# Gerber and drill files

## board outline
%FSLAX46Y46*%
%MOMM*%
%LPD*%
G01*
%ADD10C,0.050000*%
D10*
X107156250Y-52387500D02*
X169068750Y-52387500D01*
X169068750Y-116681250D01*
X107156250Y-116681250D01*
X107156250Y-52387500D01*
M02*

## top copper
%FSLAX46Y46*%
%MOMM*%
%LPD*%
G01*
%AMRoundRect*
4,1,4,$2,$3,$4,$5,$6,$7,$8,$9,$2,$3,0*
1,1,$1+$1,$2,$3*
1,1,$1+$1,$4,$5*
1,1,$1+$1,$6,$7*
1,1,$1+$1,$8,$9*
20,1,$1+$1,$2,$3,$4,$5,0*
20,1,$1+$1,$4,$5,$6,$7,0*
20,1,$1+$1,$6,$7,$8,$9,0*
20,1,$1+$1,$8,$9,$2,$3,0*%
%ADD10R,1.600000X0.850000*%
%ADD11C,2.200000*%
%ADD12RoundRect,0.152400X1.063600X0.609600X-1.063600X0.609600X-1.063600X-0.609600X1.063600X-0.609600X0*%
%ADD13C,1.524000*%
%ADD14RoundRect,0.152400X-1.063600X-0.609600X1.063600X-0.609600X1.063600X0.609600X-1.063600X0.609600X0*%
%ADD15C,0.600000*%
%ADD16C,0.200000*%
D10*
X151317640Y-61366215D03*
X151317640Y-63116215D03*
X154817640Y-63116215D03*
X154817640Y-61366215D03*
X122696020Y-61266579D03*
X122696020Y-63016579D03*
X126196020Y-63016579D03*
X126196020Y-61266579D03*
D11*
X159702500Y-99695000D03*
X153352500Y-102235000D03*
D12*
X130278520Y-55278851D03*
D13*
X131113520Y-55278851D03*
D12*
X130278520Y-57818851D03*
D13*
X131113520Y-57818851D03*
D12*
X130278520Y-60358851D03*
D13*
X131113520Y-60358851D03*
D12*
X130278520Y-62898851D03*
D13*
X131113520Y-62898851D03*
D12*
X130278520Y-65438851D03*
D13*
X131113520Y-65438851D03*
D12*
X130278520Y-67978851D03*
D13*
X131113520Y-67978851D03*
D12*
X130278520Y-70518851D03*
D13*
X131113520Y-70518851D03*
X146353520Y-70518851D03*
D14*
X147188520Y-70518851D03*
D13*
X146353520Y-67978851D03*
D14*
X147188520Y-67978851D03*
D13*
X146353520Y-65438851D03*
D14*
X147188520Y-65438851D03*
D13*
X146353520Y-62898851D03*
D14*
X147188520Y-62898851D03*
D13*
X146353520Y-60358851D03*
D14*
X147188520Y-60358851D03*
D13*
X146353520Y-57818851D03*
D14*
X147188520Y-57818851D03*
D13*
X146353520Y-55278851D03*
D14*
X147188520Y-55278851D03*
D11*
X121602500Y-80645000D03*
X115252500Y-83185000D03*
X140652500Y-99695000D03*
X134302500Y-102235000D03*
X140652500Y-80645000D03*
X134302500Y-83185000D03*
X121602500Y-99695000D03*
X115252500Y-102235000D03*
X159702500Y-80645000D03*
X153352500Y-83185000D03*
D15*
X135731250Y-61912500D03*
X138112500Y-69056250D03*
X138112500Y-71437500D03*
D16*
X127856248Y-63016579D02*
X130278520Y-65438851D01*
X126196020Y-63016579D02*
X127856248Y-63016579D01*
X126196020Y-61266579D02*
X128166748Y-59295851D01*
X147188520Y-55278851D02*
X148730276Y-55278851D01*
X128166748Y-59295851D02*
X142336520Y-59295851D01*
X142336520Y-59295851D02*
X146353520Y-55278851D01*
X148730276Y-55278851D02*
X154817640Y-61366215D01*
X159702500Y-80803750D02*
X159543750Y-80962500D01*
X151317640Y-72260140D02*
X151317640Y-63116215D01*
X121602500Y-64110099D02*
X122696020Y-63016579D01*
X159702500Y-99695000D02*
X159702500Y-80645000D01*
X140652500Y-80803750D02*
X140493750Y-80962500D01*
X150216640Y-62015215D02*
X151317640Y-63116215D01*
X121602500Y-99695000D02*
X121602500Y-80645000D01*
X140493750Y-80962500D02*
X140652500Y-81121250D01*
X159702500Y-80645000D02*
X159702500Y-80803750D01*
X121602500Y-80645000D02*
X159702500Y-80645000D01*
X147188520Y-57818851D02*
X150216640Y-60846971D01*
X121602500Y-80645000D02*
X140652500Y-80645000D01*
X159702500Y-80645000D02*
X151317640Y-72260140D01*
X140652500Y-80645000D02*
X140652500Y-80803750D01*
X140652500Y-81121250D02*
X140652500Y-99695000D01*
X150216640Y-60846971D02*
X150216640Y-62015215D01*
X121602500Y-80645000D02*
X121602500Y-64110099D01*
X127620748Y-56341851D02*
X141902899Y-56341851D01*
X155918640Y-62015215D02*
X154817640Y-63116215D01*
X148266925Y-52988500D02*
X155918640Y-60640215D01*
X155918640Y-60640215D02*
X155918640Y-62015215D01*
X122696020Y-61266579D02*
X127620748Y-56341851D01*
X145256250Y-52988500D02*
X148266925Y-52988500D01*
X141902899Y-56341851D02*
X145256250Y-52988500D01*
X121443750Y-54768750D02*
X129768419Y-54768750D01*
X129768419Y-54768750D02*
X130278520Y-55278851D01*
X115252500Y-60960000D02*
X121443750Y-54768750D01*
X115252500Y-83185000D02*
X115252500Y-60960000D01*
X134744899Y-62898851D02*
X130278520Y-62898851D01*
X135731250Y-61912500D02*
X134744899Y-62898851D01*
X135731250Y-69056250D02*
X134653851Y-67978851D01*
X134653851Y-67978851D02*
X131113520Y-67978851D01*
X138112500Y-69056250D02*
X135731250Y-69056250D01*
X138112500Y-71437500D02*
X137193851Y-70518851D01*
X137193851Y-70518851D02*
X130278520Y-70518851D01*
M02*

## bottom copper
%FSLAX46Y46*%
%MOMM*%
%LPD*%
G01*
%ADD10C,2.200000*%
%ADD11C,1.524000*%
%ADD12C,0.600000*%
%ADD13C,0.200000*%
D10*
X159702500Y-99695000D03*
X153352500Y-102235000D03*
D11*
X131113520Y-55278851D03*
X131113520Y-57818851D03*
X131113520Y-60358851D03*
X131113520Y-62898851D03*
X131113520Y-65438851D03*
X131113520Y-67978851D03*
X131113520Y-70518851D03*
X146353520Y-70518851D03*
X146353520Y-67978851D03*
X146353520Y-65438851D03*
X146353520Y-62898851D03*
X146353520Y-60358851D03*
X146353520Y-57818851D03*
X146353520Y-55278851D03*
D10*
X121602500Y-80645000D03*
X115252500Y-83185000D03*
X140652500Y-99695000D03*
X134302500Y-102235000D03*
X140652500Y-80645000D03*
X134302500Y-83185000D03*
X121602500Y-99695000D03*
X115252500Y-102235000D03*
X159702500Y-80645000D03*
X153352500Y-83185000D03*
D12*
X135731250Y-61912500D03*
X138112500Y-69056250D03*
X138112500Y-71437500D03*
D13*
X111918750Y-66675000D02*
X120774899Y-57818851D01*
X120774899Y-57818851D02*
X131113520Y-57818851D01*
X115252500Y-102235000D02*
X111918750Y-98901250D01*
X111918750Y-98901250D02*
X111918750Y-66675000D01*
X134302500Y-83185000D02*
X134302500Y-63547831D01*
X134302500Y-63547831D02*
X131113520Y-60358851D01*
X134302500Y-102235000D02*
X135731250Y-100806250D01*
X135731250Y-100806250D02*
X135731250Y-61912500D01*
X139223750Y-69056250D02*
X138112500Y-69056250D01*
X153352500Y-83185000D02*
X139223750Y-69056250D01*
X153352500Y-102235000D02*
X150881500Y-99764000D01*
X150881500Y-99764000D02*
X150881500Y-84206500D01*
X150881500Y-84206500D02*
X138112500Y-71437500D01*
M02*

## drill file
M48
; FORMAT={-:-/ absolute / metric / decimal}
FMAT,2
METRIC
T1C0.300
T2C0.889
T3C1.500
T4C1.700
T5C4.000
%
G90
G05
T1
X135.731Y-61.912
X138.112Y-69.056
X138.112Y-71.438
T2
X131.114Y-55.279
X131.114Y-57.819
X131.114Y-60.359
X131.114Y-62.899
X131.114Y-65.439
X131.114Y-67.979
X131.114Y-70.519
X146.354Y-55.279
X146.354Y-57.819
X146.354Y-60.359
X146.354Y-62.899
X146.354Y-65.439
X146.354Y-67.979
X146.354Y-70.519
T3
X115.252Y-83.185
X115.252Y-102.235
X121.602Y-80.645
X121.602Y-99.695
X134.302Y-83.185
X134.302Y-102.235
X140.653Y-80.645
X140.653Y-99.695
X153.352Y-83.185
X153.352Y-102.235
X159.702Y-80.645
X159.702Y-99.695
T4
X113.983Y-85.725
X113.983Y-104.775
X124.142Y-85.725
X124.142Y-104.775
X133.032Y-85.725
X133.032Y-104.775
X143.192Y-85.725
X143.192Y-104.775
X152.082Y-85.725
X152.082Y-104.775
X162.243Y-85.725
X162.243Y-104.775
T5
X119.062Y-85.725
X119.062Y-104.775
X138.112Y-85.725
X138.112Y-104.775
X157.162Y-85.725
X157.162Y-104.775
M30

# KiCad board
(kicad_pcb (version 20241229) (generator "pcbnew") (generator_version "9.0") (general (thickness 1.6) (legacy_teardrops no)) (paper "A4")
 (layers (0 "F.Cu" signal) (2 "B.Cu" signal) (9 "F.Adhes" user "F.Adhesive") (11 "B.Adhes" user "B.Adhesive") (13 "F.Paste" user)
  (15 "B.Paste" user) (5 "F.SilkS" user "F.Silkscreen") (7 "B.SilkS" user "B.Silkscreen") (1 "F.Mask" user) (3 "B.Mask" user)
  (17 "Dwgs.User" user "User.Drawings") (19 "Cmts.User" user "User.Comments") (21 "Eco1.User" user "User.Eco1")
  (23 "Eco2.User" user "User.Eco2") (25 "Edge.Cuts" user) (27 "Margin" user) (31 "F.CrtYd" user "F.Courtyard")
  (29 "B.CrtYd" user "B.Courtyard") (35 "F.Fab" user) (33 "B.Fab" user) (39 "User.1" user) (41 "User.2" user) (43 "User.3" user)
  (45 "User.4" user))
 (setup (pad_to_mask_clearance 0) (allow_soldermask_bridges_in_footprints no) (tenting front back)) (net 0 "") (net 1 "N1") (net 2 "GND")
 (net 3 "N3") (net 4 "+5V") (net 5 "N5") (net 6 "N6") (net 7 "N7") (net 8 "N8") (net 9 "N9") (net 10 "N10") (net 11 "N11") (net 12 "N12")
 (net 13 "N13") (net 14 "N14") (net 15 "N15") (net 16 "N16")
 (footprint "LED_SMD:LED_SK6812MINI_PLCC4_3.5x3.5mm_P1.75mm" (layer "F.Cu") (at 153.06764 62.241215)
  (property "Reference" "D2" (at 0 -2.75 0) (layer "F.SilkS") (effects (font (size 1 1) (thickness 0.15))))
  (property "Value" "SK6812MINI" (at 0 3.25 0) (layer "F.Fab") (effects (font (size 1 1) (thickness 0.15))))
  (pad "1" smd rect (at -1.75 -0.875) (size 1.6 0.85) (layers "F.Cu" "F.Mask" "F.Paste") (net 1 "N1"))
  (pad "2" smd rect (at -1.75 0.875) (size 1.6 0.85) (layers "F.Cu" "F.Mask" "F.Paste") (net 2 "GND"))
  (pad "3" smd rect (at 1.75 0.875) (size 1.6 0.85) (layers "F.Cu" "F.Mask" "F.Paste") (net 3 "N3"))
  (pad "4" smd rect (at 1.75 -0.875) (size 1.6 0.85) (layers "F.Cu" "F.Mask" "F.Paste") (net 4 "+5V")))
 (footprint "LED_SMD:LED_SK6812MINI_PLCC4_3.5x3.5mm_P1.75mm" (layer "F.Cu") (at 124.44602 62.141579)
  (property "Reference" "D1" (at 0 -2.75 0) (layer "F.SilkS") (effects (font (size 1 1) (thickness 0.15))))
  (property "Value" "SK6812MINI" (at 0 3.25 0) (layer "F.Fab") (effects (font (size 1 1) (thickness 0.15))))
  (pad "1" smd rect (at -1.75 -0.875) (size 1.6 0.85) (layers "F.Cu" "F.Mask" "F.Paste") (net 3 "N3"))
  (pad "2" smd rect (at -1.75 0.875) (size 1.6 0.85) (layers "F.Cu" "F.Mask" "F.Paste") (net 2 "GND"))
  (pad "3" smd rect (at 1.75 0.875) (size 1.6 0.85) (layers "F.Cu" "F.Mask" "F.Paste") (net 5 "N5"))
  (pad "4" smd rect (at 1.75 -0.875) (size 1.6 0.85) (layers "F.Cu" "F.Mask" "F.Paste") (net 4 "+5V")))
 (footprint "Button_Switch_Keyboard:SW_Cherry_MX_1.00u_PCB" (layer "F.Cu") (at 159.7025 99.695)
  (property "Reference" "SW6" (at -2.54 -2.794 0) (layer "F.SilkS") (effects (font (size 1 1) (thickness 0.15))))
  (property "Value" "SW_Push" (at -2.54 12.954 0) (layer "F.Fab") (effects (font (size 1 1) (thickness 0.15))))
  (pad "" np_thru_hole circle (at -7.62 5.08) (size 1.7 1.7) (drill 1.7) (layers "*.Cu" "*.Mask"))
  (pad "" np_thru_hole circle (at -2.54 5.08) (size 4 4) (drill 4) (layers "*.Cu" "*.Mask"))
  (pad "" np_thru_hole circle (at 2.54 5.08) (size 1.7 1.7) (drill 1.7) (layers "*.Cu" "*.Mask"))
  (pad "1" thru_hole circle (at 0 0) (size 2.2 2.2) (drill 1.5) (layers "*.Cu" "*.Mask") (remove_unused_layers no) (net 2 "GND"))
  (pad "2" thru_hole circle (at -6.35 2.54) (size 2.2 2.2) (drill 1.5) (layers "*.Cu" "*.Mask") (remove_unused_layers no) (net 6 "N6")))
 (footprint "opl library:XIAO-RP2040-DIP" (layer "F.Cu") (at 138.73352 62.898851)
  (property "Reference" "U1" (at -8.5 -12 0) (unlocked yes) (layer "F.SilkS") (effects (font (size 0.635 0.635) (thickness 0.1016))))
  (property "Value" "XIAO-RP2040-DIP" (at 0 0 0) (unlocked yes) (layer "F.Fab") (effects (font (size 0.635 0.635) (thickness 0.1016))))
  (pad "1" smd roundrect (at -8.455 -7.62 180) (size 2.432 1.524) (layers "F.Cu" "F.Mask") (roundrect_rratio 0.1) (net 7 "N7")
   (thermal_bridge_angle 45))
  (pad "1" thru_hole circle (at -7.62 -7.62 180) (size 1.524 1.524) (drill 0.889) (layers "*.Cu" "*.Mask") (remove_unused_layers no)
   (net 7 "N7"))
  (pad "2" smd roundrect (at -8.455 -5.08 180) (size 2.432 1.524) (layers "F.Cu" "F.Mask") (roundrect_rratio 0.1) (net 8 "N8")
   (thermal_bridge_angle 45))
  (pad "2" thru_hole circle (at -7.62 -5.08 180) (size 1.524 1.524) (drill 0.889) (layers "*.Cu" "*.Mask") (remove_unused_layers no)
   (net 8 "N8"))
  (pad "3" smd roundrect (at -8.455 -2.54 180) (size 2.432 1.524) (layers "F.Cu" "F.Mask") (roundrect_rratio 0.1) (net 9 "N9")
   (thermal_bridge_angle 45))
  (pad "3" thru_hole circle (at -7.62 -2.54 180) (size 1.524 1.524) (drill 0.889) (layers "*.Cu" "*.Mask") (remove_unused_layers no)
   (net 9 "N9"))
  (pad "4" smd roundrect (at -8.455 0 180) (size 2.432 1.524) (layers "F.Cu" "F.Mask") (roundrect_rratio 0.1) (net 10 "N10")
   (thermal_bridge_angle 45))
  (pad "4" thru_hole circle (at -7.62 0 180) (size 1.524 1.524) (drill 0.889) (layers "*.Cu" "*.Mask") (remove_unused_layers no)
   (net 10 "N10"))
  (pad "5" smd roundrect (at -8.455 2.54 180) (size 2.432 1.524) (layers "F.Cu" "F.Mask") (roundrect_rratio 0.1) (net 5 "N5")
   (thermal_bridge_angle 45))
  (pad "5" thru_hole circle (at -7.62 2.54 180) (size 1.524 1.524) (drill 0.889) (layers "*.Cu" "*.Mask") (remove_unused_layers no)
   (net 5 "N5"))
  (pad "6" smd roundrect (at -8.455 5.08 180) (size 2.432 1.524) (layers "F.Cu" "F.Mask") (roundrect_rratio 0.1) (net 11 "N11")
   (thermal_bridge_angle 45))
  (pad "6" thru_hole circle (at -7.62 5.08 180) (size 1.524 1.524) (drill 0.889) (layers "*.Cu" "*.Mask") (remove_unused_layers no)
   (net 11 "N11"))
  (pad "7" smd roundrect (at -8.455 7.62 180) (size 2.432 1.524) (layers "F.Cu" "F.Mask") (roundrect_rratio 0.1) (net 6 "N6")
   (thermal_bridge_angle 45))
  (pad "7" thru_hole circle (at -7.62 7.62 180) (size 1.524 1.524) (drill 0.889) (layers "*.Cu" "*.Mask") (remove_unused_layers no)
   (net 6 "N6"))
  (pad "8" thru_hole circle (at 7.62 7.62) (size 1.524 1.524) (drill 0.889) (layers "*.Cu" "*.Mask") (remove_unused_layers no)
   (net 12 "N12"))
  (pad "8" smd roundrect (at 8.455 7.62) (size 2.432 1.524) (layers "F.Cu" "F.Mask") (roundrect_rratio 0.1) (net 12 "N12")
   (thermal_bridge_angle 45))
  (pad "9" thru_hole circle (at 7.62 5.08) (size 1.524 1.524) (drill 0.889) (layers "*.Cu" "*.Mask") (remove_unused_layers no)
   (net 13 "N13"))
  (pad "9" smd roundrect (at 8.455 5.08) (size 2.432 1.524) (layers "F.Cu" "F.Mask") (roundrect_rratio 0.1) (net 13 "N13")
   (thermal_bridge_angle 45))
  (pad "10" thru_hole circle (at 7.62 2.54) (size 1.524 1.524) (drill 0.889) (layers "*.Cu" "*.Mask") (remove_unused_layers no)
   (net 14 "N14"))
  (pad "10" smd roundrect (at 8.455 2.54) (size 2.432 1.524) (layers "F.Cu" "F.Mask") (roundrect_rratio 0.1) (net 14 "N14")
   (thermal_bridge_angle 45))
  (pad "11" thru_hole circle (at 7.62 0) (size 1.524 1.524) (drill 0.889) (layers "*.Cu" "*.Mask") (remove_unused_layers no) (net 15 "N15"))
  (pad "11" smd roundrect (at 8.455 0) (size 2.432 1.524) (layers "F.Cu" "F.Mask") (roundrect_rratio 0.1) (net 15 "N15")
   (thermal_bridge_angle 45))
  (pad "12" thru_hole circle (at 7.62 -2.54) (size 1.524 1.524) (drill 0.889) (layers "*.Cu" "*.Mask") (remove_unused_layers no)
   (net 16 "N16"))
  (pad "12" smd roundrect (at 8.455 -2.54) (size 2.432 1.524) (layers "F.Cu" "F.Mask") (roundrect_rratio 0.1) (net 16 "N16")
   (thermal_bridge_angle 45))
  (pad "13" thru_hole circle (at 7.62 -5.08) (size 1.524 1.524) (drill 0.889) (layers "*.Cu" "*.Mask") (remove_unused_layers no)
   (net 2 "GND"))
  (pad "13" smd roundrect (at 8.455 -5.08) (size 2.432 1.524) (layers "F.Cu" "F.Mask") (roundrect_rratio 0.1) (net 2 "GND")
   (thermal_bridge_angle 45))
  (pad "14" thru_hole circle (at 7.62 -7.62) (size 1.524 1.524) (drill 0.889) (layers "*.Cu" "*.Mask") (remove_unused_layers no)
   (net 4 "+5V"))
  (pad "14" smd roundrect (at 8.455 -7.62) (size 2.432 1.524) (layers "F.Cu" "F.Mask") (roundrect_rratio 0.1) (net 4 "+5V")
   (thermal_bridge_angle 45)))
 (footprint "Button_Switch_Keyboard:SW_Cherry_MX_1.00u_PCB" (layer "F.Cu") (at 121.6025 80.645)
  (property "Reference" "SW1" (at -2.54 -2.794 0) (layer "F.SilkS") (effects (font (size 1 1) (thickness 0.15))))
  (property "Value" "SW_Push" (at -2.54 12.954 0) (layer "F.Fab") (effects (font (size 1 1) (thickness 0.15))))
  (pad "" np_thru_hole circle (at -7.62 5.08) (size 1.7 1.7) (drill 1.7) (layers "*.Cu" "*.Mask"))
  (pad "" np_thru_hole circle (at -2.54 5.08) (size 4 4) (drill 4) (layers "*.Cu" "*.Mask"))
  (pad "" np_thru_hole circle (at 2.54 5.08) (size 1.7 1.7) (drill 1.7) (layers "*.Cu" "*.Mask"))
  (pad "1" thru_hole circle (at 0 0) (size 2.2 2.2) (drill 1.5) (layers "*.Cu" "*.Mask") (remove_unused_layers no) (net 2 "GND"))
  (pad "2" thru_hole circle (at -6.35 2.54) (size 2.2 2.2) (drill 1.5) (layers "*.Cu" "*.Mask") (remove_unused_layers no) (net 7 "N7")))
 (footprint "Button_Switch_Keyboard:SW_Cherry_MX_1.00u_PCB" (layer "F.Cu") (at 140.6525 99.695)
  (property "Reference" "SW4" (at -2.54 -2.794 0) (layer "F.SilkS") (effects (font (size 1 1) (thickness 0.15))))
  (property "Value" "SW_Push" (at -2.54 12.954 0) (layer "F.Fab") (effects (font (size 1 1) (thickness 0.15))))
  (pad "" np_thru_hole circle (at -7.62 5.08) (size 1.7 1.7) (drill 1.7) (layers "*.Cu" "*.Mask"))
  (pad "" np_thru_hole circle (at -2.54 5.08) (size 4 4) (drill 4) (layers "*.Cu" "*.Mask"))
  (pad "" np_thru_hole circle (at 2.54 5.08) (size 1.7 1.7) (drill 1.7) (layers "*.Cu" "*.Mask"))
  (pad "1" thru_hole circle (at 0 0) (size 2.2 2.2) (drill 1.5) (layers "*.Cu" "*.Mask") (remove_unused_layers no) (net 2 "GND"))
  (pad "2" thru_hole circle (at -6.35 2.54) (size 2.2 2.2) (drill 1.5) (layers "*.Cu" "*.Mask") (remove_unused_layers no) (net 10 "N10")))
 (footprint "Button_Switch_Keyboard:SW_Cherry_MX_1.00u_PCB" (layer "F.Cu") (at 140.6525 80.645)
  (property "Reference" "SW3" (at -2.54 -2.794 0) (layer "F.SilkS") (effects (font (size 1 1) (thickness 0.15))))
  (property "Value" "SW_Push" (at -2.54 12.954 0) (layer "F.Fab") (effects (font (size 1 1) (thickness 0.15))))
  (pad "" np_thru_hole circle (at -7.62 5.08) (size 1.7 1.7) (drill 1.7) (layers "*.Cu" "*.Mask"))
  (pad "" np_thru_hole circle (at -2.54 5.08) (size 4 4) (drill 4) (layers "*.Cu" "*.Mask"))
  (pad "" np_thru_hole circle (at 2.54 5.08) (size 1.7 1.7) (drill 1.7) (layers "*.Cu" "*.Mask"))
  (pad "1" thru_hole circle (at 0 0) (size 2.2 2.2) (drill 1.5) (layers "*.Cu" "*.Mask") (remove_unused_layers no) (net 2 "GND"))
  (pad "2" thru_hole circle (at -6.35 2.54) (size 2.2 2.2) (drill 1.5) (layers "*.Cu" "*.Mask") (remove_unused_layers no) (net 9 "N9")))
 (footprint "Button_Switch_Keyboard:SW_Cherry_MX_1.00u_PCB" (layer "F.Cu") (at 121.6025 99.695)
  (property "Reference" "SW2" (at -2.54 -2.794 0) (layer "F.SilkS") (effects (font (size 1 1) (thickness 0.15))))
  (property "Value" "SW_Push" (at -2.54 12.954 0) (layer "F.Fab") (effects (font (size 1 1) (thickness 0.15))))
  (pad "" np_thru_hole circle (at -7.62 5.08) (size 1.7 1.7) (drill 1.7) (layers "*.Cu" "*.Mask"))
  (pad "" np_thru_hole circle (at -2.54 5.08) (size 4 4) (drill 4) (layers "*.Cu" "*.Mask"))
  (pad "" np_thru_hole circle (at 2.54 5.08) (size 1.7 1.7) (drill 1.7) (layers "*.Cu" "*.Mask"))
  (pad "1" thru_hole circle (at 0 0) (size 2.2 2.2) (drill 1.5) (layers "*.Cu" "*.Mask") (remove_unused_layers no) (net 2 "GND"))
  (pad "2" thru_hole circle (at -6.35 2.54) (size 2.2 2.2) (drill 1.5) (layers "*.Cu" "*.Mask") (remove_unused_layers no) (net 8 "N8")))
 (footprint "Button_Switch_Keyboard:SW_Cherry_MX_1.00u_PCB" (layer "F.Cu") (at 159.7025 80.645)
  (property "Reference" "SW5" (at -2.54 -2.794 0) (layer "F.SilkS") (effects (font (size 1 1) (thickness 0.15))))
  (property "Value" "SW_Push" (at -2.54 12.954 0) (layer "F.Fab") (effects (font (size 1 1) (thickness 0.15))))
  (pad "" np_thru_hole circle (at -7.62 5.08) (size 1.7 1.7) (drill 1.7) (layers "*.Cu" "*.Mask"))
  (pad "" np_thru_hole circle (at -2.54 5.08) (size 4 4) (drill 4) (layers "*.Cu" "*.Mask"))
  (pad "" np_thru_hole circle (at 2.54 5.08) (size 1.7 1.7) (drill 1.7) (layers "*.Cu" "*.Mask"))
  (pad "1" thru_hole circle (at 0 0) (size 2.2 2.2) (drill 1.5) (layers "*.Cu" "*.Mask") (remove_unused_layers no) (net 2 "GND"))
  (pad "2" thru_hole circle (at -6.35 2.54) (size 2.2 2.2) (drill 1.5) (layers "*.Cu" "*.Mask") (remove_unused_layers no) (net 11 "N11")))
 (gr_rect (start 107.15625 52.3875) (end 169.06875 116.68125) (stroke (width 0.05) (type default)) (fill no) (layer "Edge.Cuts"))
 (segment (start 127.856248 63.016579) (end 130.27852 65.438851) (width 0.2) (layer "F.Cu") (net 5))
 (segment (start 126.19602 63.016579) (end 127.856248 63.016579) (width 0.2) (layer "F.Cu") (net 5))
 (segment (start 126.19602 61.266579) (end 128.166748 59.295851) (width 0.2) (layer "F.Cu") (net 4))
 (segment (start 147.18852 55.278851) (end 148.730276 55.278851) (width 0.2) (layer "F.Cu") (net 4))
 (segment (start 128.166748 59.295851) (end 142.33652 59.295851) (width 0.2) (layer "F.Cu") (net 4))
 (segment (start 142.33652 59.295851) (end 146.35352 55.278851) (width 0.2) (layer "F.Cu") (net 4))
 (segment (start 148.730276 55.278851) (end 154.81764 61.366215) (width 0.2) (layer "F.Cu") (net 4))
 (segment (start 159.7025 80.80375) (end 159.54375 80.9625) (width 0.2) (layer "F.Cu") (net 2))
 (segment (start 151.31764 72.26014) (end 151.31764 63.116215) (width 0.2) (layer "F.Cu") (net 2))
 (segment (start 121.6025 64.110099) (end 122.69602 63.016579) (width 0.2) (layer "F.Cu") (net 2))
 (segment (start 159.7025 99.695) (end 159.7025 80.645) (width 0.2) (layer "F.Cu") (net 2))
 (segment (start 140.6525 80.80375) (end 140.49375 80.9625) (width 0.2) (layer "F.Cu") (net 2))
 (segment (start 150.21664 62.015215) (end 151.31764 63.116215) (width 0.2) (layer "F.Cu") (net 2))
 (segment (start 121.6025 99.695) (end 121.6025 80.645) (width 0.2) (layer "F.Cu") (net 2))
 (segment (start 140.49375 80.9625) (end 140.6525 81.12125) (width 0.2) (layer "F.Cu") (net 2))
 (segment (start 159.7025 80.645) (end 159.7025 80.80375) (width 0.2) (layer "F.Cu") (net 2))
 (segment (start 121.6025 80.645) (end 159.7025 80.645) (width 0.2) (layer "F.Cu") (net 2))
 (segment (start 147.18852 57.818851) (end 150.21664 60.846971) (width 0.2) (layer "F.Cu") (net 2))
 (segment (start 121.6025 80.645) (end 140.6525 80.645) (width 0.2) (layer "F.Cu") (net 2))
 (segment (start 159.7025 80.645) (end 151.31764 72.26014) (width 0.2) (layer "F.Cu") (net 2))
 (segment (start 140.6525 80.645) (end 140.6525 80.80375) (width 0.2) (layer "F.Cu") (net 2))
 (segment (start 140.6525 81.12125) (end 140.6525 99.695) (width 0.2) (layer "F.Cu") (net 2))
 (segment (start 150.21664 60.846971) (end 150.21664 62.015215) (width 0.2) (layer "F.Cu") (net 2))
 (segment (start 121.6025 80.645) (end 121.6025 64.110099) (width 0.2) (layer "F.Cu") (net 2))
 (segment (start 127.620748 56.341851) (end 141.902899 56.341851) (width 0.2) (layer "F.Cu") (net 3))
 (segment (start 155.91864 62.015215) (end 154.81764 63.116215) (width 0.2) (layer "F.Cu") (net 3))
 (segment (start 148.266925 52.9885) (end 155.91864 60.640215) (width 0.2) (layer "F.Cu") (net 3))
 (segment (start 155.91864 60.640215) (end 155.91864 62.015215) (width 0.2) (layer "F.Cu") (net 3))
 (segment (start 122.69602 61.266579) (end 127.620748 56.341851) (width 0.2) (layer "F.Cu") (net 3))
 (segment (start 145.25625 52.9885) (end 148.266925 52.9885) (width 0.2) (layer "F.Cu") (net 3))
 (segment (start 141.902899 56.341851) (end 145.25625 52.9885) (width 0.2) (layer "F.Cu") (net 3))
 (segment (start 121.44375 54.76875) (end 129.768419 54.76875) (width 0.2) (layer "F.Cu") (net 7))
 (segment (start 129.768419 54.76875) (end 130.27852 55.278851) (width 0.2) (layer "F.Cu") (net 7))
 (segment (start 115.2525 60.96) (end 121.44375 54.76875) (width 0.2) (layer "F.Cu") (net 7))
 (segment (start 115.2525 83.185) (end 115.2525 60.96) (width 0.2) (layer "F.Cu") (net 7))
 (segment (start 111.91875 66.675) (end 120.774899 57.818851) (width 0.2) (layer "B.Cu") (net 8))
 (segment (start 120.774899 57.818851) (end 131.11352 57.818851) (width 0.2) (layer "B.Cu") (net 8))
 (segment (start 115.2525 102.235) (end 111.91875 98.90125) (width 0.2) (layer "B.Cu") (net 8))
 (segment (start 111.91875 98.90125) (end 111.91875 66.675) (width 0.2) (layer "B.Cu") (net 8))
 (segment (start 134.3025 83.185) (end 134.3025 63.547831) (width 0.2) (layer "B.Cu") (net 9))
 (segment (start 134.3025 63.547831) (end 131.11352 60.358851) (width 0.2) (layer "B.Cu") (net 9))
 (segment (start 134.744899 62.898851) (end 130.27852 62.898851) (width 0.2) (layer "F.Cu") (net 10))
 (segment (start 135.73125 61.9125) (end 134.744899 62.898851) (width 0.2) (layer "F.Cu") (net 10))
 (via (at 135.73125 61.9125) (size 0.6) (drill 0.3) (layers "F.Cu" "B.Cu") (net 10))
 (segment (start 134.3025 102.235) (end 135.73125 100.80625) (width 0.2) (layer "B.Cu") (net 10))
 (segment (start 135.73125 100.80625) (end 135.73125 61.9125) (width 0.2) (layer "B.Cu") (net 10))
 (segment (start 135.73125 69.05625) (end 134.653851 67.978851) (width 0.2) (layer "F.Cu") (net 11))
 (segment (start 134.653851 67.978851) (end 131.11352 67.978851) (width 0.2) (layer "F.Cu") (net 11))
 (segment (start 138.1125 69.05625) (end 135.73125 69.05625) (width 0.2) (layer "F.Cu") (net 11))
 (via (at 138.1125 69.05625) (size 0.6) (drill 0.3) (layers "F.Cu" "B.Cu") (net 11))
 (segment (start 139.22375 69.05625) (end 138.1125 69.05625) (width 0.2) (layer "B.Cu") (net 11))
 (segment (start 153.3525 83.185) (end 139.22375 69.05625) (width 0.2) (layer "B.Cu") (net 11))
 (segment (start 138.1125 71.4375) (end 137.193851 70.518851) (width 0.2) (layer "F.Cu") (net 6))
 (segment (start 137.193851 70.518851) (end 130.27852 70.518851) (width 0.2) (layer "F.Cu") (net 6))
 (via (at 138.1125 71.4375) (size 0.6) (drill 0.3) (layers "F.Cu" "B.Cu") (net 6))
 (segment (start 153.3525 102.235) (end 150.8815 99.764) (width 0.2) (layer "B.Cu") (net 6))
 (segment (start 150.8815 99.764) (end 150.8815 84.2065) (width 0.2) (layer "B.Cu") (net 6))
 (segment (start 150.8815 84.2065) (end 138.1125 71.4375) (width 0.2) (layer "B.Cu") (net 6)))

